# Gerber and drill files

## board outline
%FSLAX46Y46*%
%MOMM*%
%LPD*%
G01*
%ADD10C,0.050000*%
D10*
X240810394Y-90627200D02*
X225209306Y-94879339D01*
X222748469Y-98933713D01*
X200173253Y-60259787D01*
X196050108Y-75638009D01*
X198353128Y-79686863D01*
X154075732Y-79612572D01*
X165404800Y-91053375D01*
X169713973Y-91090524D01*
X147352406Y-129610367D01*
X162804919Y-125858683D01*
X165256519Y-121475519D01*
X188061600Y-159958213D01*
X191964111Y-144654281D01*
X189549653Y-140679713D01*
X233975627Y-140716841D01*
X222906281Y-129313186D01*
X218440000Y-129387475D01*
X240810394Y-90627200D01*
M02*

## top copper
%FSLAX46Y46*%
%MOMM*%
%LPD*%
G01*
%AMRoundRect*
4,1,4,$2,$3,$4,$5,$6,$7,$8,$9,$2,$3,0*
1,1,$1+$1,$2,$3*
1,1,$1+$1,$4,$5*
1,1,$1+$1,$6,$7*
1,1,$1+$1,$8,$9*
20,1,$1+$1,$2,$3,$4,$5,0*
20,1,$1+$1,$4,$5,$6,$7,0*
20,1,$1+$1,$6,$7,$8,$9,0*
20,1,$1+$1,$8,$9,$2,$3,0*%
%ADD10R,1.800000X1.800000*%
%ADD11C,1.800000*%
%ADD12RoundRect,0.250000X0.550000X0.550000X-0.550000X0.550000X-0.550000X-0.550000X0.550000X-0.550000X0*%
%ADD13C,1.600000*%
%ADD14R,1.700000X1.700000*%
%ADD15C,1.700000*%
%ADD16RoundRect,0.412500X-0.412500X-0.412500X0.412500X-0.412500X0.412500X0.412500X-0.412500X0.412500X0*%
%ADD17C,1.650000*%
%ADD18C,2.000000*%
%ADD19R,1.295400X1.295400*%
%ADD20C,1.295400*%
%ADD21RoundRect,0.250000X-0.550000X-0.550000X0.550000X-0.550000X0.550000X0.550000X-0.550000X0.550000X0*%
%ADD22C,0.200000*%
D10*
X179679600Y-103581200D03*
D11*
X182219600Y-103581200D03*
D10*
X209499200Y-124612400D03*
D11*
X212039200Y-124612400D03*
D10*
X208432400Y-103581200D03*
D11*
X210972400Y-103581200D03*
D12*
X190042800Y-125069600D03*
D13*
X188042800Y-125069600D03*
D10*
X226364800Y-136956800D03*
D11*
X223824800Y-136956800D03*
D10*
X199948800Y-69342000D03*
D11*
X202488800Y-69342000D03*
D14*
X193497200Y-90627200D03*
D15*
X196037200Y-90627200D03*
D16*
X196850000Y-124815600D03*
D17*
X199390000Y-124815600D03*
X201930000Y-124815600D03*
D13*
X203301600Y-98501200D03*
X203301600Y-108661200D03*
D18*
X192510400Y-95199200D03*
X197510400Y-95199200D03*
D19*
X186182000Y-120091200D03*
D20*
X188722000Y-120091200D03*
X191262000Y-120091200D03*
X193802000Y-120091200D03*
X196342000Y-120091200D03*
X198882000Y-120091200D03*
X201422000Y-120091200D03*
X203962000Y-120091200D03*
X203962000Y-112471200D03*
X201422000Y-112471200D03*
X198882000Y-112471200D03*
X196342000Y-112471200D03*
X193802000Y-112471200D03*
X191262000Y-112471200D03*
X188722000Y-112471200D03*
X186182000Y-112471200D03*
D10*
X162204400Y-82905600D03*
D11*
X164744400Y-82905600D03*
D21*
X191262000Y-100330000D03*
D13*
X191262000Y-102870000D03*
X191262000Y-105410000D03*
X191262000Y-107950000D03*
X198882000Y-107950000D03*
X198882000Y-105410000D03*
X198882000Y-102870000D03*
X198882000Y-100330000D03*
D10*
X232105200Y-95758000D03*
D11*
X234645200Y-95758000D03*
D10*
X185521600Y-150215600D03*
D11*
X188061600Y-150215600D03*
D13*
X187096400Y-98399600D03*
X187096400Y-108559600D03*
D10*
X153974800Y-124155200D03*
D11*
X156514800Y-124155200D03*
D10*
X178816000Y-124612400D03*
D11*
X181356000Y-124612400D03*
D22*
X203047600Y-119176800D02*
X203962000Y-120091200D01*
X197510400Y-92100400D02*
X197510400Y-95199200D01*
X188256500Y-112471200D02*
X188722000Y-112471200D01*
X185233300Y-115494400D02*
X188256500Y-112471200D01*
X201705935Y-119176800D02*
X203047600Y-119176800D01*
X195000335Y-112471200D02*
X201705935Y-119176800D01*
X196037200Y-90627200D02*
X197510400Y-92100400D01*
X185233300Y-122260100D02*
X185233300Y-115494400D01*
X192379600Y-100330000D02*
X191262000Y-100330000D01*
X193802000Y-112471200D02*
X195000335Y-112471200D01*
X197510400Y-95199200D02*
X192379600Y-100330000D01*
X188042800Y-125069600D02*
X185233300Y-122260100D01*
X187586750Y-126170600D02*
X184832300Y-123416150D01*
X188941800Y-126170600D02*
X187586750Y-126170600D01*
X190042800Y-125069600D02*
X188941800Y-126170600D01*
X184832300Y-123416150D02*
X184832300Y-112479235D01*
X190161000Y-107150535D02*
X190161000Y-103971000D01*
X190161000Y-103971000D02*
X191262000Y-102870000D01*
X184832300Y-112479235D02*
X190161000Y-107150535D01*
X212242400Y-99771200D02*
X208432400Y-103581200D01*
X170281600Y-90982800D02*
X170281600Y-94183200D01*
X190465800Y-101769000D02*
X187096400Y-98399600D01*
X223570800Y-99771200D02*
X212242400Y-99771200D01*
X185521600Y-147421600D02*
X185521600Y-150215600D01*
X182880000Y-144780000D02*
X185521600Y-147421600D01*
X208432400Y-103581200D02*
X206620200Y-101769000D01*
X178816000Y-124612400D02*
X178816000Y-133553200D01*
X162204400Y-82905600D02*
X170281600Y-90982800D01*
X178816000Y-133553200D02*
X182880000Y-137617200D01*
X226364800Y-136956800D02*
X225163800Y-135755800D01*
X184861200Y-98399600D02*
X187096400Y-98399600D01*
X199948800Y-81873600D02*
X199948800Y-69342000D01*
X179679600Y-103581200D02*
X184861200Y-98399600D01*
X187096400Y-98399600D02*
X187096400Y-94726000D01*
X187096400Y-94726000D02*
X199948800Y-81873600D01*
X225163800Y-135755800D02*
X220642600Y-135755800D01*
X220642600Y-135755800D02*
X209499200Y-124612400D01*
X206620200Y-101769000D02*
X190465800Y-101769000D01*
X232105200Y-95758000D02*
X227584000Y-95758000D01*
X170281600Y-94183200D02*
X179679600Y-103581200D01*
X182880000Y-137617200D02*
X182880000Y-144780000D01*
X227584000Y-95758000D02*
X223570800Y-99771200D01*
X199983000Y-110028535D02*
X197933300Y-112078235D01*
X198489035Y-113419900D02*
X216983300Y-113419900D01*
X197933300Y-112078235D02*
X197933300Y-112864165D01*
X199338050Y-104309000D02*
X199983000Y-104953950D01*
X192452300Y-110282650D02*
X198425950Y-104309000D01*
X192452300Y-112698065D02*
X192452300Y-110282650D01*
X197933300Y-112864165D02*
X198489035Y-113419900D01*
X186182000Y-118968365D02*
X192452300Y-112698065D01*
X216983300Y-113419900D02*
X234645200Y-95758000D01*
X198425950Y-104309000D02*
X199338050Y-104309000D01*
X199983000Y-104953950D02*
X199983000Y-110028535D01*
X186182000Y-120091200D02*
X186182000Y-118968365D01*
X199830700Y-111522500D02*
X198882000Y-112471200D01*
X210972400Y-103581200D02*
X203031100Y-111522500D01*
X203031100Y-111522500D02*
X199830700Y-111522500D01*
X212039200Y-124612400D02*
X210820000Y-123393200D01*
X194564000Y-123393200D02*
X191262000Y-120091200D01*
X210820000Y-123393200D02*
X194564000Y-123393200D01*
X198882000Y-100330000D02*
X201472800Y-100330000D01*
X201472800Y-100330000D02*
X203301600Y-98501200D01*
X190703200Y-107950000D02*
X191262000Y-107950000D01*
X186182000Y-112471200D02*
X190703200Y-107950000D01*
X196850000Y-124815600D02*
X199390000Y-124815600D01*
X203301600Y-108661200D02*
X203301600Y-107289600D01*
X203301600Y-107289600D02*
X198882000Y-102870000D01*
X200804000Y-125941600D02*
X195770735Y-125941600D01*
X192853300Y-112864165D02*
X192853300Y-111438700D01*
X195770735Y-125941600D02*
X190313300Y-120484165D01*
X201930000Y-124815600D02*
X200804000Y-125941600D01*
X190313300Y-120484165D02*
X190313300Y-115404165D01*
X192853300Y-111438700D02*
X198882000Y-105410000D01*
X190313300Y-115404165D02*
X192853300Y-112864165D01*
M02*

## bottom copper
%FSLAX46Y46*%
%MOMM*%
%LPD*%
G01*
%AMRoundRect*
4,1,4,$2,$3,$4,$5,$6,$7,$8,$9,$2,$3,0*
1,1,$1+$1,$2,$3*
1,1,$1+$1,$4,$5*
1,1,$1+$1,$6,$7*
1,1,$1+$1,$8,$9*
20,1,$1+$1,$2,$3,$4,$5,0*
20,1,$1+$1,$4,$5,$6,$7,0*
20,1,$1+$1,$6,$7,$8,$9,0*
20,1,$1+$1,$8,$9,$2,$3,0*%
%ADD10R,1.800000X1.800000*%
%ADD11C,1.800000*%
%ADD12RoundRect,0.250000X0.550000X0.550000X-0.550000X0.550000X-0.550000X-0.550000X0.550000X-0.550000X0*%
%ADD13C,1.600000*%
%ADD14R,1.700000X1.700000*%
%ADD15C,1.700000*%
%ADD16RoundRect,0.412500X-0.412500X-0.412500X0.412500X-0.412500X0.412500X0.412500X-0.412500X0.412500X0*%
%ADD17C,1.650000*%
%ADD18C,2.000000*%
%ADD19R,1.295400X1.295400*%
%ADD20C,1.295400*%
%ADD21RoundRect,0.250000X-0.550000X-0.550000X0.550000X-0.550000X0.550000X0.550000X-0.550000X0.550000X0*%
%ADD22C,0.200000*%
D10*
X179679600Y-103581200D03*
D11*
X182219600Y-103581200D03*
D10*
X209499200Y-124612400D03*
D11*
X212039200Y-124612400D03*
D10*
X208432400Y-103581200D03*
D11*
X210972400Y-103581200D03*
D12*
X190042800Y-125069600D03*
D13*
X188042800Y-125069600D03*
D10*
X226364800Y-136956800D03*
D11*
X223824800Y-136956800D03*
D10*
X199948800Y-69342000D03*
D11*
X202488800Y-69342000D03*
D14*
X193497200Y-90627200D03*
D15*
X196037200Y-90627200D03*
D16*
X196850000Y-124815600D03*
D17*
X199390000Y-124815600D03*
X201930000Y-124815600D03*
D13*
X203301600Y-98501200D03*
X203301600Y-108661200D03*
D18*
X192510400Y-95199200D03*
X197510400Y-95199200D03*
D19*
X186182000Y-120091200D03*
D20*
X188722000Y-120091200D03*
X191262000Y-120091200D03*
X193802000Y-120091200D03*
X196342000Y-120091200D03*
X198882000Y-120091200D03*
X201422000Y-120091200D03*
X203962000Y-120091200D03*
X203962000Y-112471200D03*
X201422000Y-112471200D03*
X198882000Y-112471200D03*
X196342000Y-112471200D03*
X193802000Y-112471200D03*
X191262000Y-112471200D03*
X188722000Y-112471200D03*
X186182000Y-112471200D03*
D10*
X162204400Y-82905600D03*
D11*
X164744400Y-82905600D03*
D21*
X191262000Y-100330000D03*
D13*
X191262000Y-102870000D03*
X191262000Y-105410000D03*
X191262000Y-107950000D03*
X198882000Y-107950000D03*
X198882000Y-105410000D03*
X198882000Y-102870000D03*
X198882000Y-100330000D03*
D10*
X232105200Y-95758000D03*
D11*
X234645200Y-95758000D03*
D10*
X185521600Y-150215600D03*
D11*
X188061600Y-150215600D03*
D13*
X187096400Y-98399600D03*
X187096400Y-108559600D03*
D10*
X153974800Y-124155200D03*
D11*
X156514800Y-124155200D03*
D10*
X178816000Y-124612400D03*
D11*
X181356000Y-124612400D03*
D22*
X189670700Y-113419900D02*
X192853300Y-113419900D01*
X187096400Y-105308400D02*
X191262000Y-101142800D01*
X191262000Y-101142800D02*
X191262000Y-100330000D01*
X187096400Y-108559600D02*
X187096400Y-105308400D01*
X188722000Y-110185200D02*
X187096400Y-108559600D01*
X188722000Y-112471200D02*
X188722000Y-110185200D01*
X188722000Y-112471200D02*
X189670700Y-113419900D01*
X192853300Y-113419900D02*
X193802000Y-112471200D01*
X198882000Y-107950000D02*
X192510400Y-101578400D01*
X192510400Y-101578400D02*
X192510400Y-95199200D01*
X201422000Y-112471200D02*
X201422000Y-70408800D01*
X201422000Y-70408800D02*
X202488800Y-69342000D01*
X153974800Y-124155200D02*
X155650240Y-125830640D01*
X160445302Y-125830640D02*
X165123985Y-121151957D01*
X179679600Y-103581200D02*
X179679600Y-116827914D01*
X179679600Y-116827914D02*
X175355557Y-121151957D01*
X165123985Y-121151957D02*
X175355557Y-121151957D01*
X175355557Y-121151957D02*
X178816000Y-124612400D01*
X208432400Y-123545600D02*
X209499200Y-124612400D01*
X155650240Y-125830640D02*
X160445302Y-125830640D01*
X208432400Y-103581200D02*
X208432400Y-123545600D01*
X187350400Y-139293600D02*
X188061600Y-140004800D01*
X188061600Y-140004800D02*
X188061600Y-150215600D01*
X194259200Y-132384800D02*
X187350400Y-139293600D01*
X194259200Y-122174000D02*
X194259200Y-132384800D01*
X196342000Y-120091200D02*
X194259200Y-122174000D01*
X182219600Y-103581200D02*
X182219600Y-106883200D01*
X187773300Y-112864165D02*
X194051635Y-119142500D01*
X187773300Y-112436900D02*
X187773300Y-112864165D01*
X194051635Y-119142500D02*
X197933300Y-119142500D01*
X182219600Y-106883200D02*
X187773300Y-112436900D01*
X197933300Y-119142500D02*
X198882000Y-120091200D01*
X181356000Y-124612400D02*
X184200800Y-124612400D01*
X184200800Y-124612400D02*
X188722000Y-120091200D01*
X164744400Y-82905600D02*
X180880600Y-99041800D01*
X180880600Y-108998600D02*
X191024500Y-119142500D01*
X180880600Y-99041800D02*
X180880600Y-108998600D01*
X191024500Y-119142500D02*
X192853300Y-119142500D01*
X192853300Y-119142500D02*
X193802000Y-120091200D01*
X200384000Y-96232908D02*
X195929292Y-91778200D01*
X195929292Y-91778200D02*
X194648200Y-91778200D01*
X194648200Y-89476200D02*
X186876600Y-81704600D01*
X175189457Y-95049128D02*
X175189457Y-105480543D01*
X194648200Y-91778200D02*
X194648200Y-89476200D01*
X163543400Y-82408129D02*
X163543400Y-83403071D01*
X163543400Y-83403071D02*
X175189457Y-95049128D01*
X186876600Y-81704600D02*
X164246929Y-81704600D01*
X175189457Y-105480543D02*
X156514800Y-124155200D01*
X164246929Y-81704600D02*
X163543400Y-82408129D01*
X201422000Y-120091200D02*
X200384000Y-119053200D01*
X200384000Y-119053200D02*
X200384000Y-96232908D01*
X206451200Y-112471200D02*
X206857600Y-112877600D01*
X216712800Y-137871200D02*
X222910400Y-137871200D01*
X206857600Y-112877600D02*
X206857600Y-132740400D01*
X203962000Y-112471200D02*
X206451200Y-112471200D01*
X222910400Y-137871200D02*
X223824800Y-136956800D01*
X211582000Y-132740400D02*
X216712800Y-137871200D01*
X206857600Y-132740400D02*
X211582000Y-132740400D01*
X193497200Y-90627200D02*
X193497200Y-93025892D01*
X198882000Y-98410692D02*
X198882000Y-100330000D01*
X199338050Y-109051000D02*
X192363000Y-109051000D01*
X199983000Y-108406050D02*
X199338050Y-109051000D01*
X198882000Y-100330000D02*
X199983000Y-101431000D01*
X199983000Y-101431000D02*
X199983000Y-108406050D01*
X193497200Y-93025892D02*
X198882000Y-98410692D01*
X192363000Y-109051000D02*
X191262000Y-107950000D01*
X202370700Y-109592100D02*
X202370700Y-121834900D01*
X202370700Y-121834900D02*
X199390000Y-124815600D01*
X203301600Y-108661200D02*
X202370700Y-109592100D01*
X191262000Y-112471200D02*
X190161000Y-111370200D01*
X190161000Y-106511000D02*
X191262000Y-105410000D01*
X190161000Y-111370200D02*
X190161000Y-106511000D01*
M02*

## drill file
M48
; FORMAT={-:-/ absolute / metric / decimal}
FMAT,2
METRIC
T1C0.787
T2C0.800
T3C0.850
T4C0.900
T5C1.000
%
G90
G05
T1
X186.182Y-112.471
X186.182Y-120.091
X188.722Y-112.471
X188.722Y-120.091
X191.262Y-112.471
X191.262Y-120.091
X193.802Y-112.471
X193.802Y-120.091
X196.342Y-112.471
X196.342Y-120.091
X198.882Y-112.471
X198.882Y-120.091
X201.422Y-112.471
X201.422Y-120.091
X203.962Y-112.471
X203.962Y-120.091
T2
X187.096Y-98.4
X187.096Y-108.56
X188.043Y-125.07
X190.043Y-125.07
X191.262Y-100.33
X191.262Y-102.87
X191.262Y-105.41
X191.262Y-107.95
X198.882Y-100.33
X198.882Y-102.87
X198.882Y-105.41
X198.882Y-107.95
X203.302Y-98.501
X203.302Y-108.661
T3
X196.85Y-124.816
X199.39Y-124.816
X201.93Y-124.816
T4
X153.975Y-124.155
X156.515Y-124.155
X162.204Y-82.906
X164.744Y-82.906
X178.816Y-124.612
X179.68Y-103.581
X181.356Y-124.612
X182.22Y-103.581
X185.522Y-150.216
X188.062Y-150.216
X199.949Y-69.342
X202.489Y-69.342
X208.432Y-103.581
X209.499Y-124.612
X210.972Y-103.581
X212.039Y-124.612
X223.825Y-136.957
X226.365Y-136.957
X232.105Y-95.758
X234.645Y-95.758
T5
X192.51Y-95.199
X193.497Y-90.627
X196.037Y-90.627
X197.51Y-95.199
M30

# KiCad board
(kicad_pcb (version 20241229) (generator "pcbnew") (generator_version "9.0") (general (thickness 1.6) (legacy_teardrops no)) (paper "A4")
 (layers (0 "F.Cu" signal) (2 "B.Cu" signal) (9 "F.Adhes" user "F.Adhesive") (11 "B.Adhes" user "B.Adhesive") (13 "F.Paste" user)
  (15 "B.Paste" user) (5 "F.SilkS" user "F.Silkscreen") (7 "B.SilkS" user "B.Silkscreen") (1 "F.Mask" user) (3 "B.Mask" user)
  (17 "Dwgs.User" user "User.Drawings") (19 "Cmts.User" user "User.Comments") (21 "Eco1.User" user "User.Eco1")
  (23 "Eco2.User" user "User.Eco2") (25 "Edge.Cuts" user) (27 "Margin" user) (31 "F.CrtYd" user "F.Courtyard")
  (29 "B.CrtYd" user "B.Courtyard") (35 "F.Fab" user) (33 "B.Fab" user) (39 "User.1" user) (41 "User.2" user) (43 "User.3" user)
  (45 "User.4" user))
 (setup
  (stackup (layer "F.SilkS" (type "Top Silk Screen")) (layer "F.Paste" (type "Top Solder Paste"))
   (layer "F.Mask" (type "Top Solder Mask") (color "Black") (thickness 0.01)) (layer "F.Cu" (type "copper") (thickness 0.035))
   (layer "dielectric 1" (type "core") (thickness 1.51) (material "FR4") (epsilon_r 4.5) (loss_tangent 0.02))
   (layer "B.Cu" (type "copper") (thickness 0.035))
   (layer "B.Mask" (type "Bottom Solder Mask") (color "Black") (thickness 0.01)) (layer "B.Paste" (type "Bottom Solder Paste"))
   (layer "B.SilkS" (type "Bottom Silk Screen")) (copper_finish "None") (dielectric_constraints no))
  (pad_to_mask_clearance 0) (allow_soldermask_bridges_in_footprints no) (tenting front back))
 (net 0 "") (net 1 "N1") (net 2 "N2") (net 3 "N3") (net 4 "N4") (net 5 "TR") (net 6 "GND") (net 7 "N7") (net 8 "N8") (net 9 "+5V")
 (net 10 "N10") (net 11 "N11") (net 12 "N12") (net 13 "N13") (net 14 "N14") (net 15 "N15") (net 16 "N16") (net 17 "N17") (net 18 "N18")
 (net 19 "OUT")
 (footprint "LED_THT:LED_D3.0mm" (layer "F.Cu") (at 179.6796 103.5812)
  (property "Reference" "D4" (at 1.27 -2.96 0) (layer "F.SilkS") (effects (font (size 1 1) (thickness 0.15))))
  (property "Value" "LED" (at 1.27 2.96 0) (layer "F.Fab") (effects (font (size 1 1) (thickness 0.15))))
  (pad "1" thru_hole rect (at 0 0) (size 1.8 1.8) (drill 0.9) (layers "*.Cu" "*.Mask") (remove_unused_layers no) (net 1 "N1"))
  (pad "2" thru_hole circle (at 2.54 0) (size 1.8 1.8) (drill 0.9) (layers "*.Cu" "*.Mask") (remove_unused_layers no) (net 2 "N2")))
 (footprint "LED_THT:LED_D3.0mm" (layer "F.Cu") (at 209.4992 124.6124)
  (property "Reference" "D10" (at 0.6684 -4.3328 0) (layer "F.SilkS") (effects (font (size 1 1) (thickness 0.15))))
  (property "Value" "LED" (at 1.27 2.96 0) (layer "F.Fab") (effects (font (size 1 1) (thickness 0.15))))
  (pad "1" thru_hole rect (at 0 0) (size 1.8 1.8) (drill 0.9) (layers "*.Cu" "*.Mask") (remove_unused_layers no) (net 1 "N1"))
  (pad "2" thru_hole circle (at 2.54 0) (size 1.8 1.8) (drill 0.9) (layers "*.Cu" "*.Mask") (remove_unused_layers no) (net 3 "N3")))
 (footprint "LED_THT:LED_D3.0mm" (layer "F.Cu") (at 208.4324 103.5812)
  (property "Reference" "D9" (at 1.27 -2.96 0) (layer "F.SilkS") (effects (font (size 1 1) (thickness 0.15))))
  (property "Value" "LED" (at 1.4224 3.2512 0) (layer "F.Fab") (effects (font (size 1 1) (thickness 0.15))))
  (pad "1" thru_hole rect (at 0 0) (size 1.8 1.8) (drill 0.9) (layers "*.Cu" "*.Mask") (remove_unused_layers no) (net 1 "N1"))
  (pad "2" thru_hole circle (at 2.54 0) (size 1.8 1.8) (drill 0.9) (layers "*.Cu" "*.Mask") (remove_unused_layers no) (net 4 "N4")))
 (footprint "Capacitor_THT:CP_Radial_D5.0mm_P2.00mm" (layer "F.Cu") (at 190.0428 125.0696 180)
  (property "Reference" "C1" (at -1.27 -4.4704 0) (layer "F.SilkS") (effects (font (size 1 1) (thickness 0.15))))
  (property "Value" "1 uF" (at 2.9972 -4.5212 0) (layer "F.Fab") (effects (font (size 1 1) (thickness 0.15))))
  (pad "1" thru_hole roundrect (at 0 0 180) (size 1.6 1.6) (drill 0.8) (layers "*.Cu" "*.Mask") (remove_unused_layers no)
   (roundrect_rratio 0.15625) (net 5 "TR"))
  (pad "2" thru_hole circle (at 2 0 180) (size 1.6 1.6) (drill 0.8) (layers "*.Cu" "*.Mask") (remove_unused_layers no) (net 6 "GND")))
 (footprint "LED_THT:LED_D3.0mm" (layer "F.Cu") (at 226.3648 136.9568 180)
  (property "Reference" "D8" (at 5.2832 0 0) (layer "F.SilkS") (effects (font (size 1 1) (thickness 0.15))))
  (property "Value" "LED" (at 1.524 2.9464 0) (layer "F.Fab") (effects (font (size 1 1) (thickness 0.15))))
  (pad "1" thru_hole rect (at 0 0 180) (size 1.8 1.8) (drill 0.9) (layers "*.Cu" "*.Mask") (remove_unused_layers no) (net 1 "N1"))
  (pad "2" thru_hole circle (at 2.54 0 180) (size 1.8 1.8) (drill 0.9) (layers "*.Cu" "*.Mask") (remove_unused_layers no) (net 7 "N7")))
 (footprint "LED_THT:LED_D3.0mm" (layer "F.Cu") (at 199.9488 69.342)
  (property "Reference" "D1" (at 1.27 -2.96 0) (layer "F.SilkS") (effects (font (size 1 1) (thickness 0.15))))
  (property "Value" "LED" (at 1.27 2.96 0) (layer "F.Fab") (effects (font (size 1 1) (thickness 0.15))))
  (pad "1" thru_hole rect (at 0 0) (size 1.8 1.8) (drill 0.9) (layers "*.Cu" "*.Mask") (remove_unused_layers no) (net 1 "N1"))
  (pad "2" thru_hole circle (at 2.54 0) (size 1.8 1.8) (drill 0.9) (layers "*.Cu" "*.Mask") (remove_unused_layers no) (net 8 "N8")))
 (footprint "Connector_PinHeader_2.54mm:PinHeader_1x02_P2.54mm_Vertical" (layer "F.Cu") (at 193.4972 90.6272 90)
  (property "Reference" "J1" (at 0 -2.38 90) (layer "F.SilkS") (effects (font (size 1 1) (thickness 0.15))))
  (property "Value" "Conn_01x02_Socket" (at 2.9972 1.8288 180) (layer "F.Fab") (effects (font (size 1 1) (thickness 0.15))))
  (pad "1" thru_hole rect (at 0 0 90) (size 1.7 1.7) (drill 1) (layers "*.Cu" "*.Mask") (remove_unused_layers no) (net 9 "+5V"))
  (pad "2" thru_hole circle (at 0 2.54 90) (size 1.7 1.7) (drill 1) (layers "*.Cu" "*.Mask") (remove_unused_layers no) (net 6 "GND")))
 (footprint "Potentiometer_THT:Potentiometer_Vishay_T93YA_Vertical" (layer "F.Cu") (at 196.85 124.8156)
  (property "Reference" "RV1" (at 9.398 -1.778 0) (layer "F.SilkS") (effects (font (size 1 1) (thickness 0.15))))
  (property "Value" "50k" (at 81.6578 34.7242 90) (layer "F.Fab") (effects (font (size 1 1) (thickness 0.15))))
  (pad "1" thru_hole roundrect (at 0 0) (size 1.65 1.65) (drill 0.85) (layers "*.Cu" "*.Mask") (remove_unused_layers no)
   (roundrect_rratio 0.25) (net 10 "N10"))
  (pad "2" thru_hole circle (at 2.54 0) (size 1.65 1.65) (drill 0.85) (layers "*.Cu" "*.Mask") (remove_unused_layers no) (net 10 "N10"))
  (pad "3" thru_hole circle (at 5.08 0) (size 1.65 1.65) (drill 0.85) (layers "*.Cu" "*.Mask") (remove_unused_layers no) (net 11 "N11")))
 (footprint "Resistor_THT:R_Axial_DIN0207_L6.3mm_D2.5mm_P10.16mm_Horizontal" (layer "F.Cu") (at 203.3016 98.5012 -90)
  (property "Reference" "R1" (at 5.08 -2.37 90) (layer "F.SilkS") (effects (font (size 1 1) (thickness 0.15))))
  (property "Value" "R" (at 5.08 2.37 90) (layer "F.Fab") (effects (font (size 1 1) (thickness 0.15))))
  (pad "1" thru_hole circle (at 0 0 270) (size 1.6 1.6) (drill 0.8) (layers "*.Cu" "*.Mask") (remove_unused_layers no) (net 9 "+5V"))
  (pad "2" thru_hole circle (at 10.16 0 270) (size 1.6 1.6) (drill 0.8) (layers "*.Cu" "*.Mask") (remove_unused_layers no) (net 10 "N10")))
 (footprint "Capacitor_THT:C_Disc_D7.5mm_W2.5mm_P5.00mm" (layer "F.Cu") (at 192.5104 95.1992)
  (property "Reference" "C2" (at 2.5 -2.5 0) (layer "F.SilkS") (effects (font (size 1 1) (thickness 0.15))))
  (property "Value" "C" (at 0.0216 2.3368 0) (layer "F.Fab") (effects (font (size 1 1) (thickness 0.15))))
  (pad "1" thru_hole circle (at 0 0) (size 2 2) (drill 1) (layers "*.Cu" "*.Mask") (remove_unused_layers no) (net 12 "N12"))
  (pad "2" thru_hole circle (at 5 0) (size 2 2) (drill 1) (layers "*.Cu" "*.Mask") (remove_unused_layers no) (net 6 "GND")))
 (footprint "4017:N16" (layer "F.Cu") (at 203.962 112.4712 90)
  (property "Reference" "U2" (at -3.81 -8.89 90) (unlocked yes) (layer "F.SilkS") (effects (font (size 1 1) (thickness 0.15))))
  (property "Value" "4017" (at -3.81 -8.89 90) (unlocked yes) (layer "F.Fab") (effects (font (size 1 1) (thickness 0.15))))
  (pad "1" thru_hole rect (at -7.62 -17.78 90) (size 1.2954 1.2954) (drill 0.7874) (layers "*.Cu" "*.Mask") (remove_unused_layers no)
   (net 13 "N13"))
  (pad "2" thru_hole circle (at -7.62 -15.24 90) (size 1.2954 1.2954) (drill 0.7874) (layers "*.Cu" "*.Mask") (remove_unused_layers no)
   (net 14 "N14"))
  (pad "3" thru_hole circle (at -7.62 -12.7 90) (size 1.2954 1.2954) (drill 0.7874) (layers "*.Cu" "*.Mask") (remove_unused_layers no)
   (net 3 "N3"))
  (pad "4" thru_hole circle (at -7.62 -10.16 90) (size 1.2954 1.2954) (drill 0.7874) (layers "*.Cu" "*.Mask") (remove_unused_layers no)
   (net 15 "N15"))
  (pad "5" thru_hole circle (at -7.62 -7.62 90) (size 1.2954 1.2954) (drill 0.7874) (layers "*.Cu" "*.Mask") (remove_unused_layers no)
   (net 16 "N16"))
  (pad "6" thru_hole circle (at -7.62 -5.08 90) (size 1.2954 1.2954) (drill 0.7874) (layers "*.Cu" "*.Mask") (remove_unused_layers no)
   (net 2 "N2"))
  (pad "7" thru_hole circle (at -7.62 -2.54 90) (size 1.2954 1.2954) (drill 0.7874) (layers "*.Cu" "*.Mask") (remove_unused_layers no)
   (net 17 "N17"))
  (pad "8" thru_hole circle (at -7.62 0 90) (size 1.2954 1.2954) (drill 0.7874) (layers "*.Cu" "*.Mask") (remove_unused_layers no)
   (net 6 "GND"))
  (pad "9" thru_hole circle (at 0 0 90) (size 1.2954 1.2954) (drill 0.7874) (layers "*.Cu" "*.Mask") (remove_unused_layers no) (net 7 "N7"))
  (pad "10" thru_hole circle (at 0 -2.54 90) (size 1.2954 1.2954) (drill 0.7874) (layers "*.Cu" "*.Mask") (remove_unused_layers no)
   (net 8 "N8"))
  (pad "11" thru_hole circle (at 0 -5.08 90) (size 1.2954 1.2954) (drill 0.7874) (layers "*.Cu" "*.Mask") (remove_unused_layers no)
   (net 4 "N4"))
  (pad "12" thru_hole circle (at 0 -7.62 90) (size 1.2954 1.2954) (drill 0.7874) (layers "*.Cu" "*.Mask") (remove_unused_layers no)
   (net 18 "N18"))
  (pad "13" thru_hole circle (at 0 -10.16 90) (size 1.2954 1.2954) (drill 0.7874) (layers "*.Cu" "*.Mask") (remove_unused_layers no)
   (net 6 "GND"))
  (pad "14" thru_hole circle (at 0 -12.7 90) (size 1.2954 1.2954) (drill 0.7874) (layers "*.Cu" "*.Mask") (remove_unused_layers no)
   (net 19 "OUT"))
  (pad "15" thru_hole circle (at 0 -15.24 90) (size 1.2954 1.2954) (drill 0.7874) (layers "*.Cu" "*.Mask") (remove_unused_layers no)
   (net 6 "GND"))
  (pad "16" thru_hole circle (at 0 -17.78 90) (size 1.2954 1.2954) (drill 0.7874) (layers "*.Cu" "*.Mask") (remove_unused_layers no)
   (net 9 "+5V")))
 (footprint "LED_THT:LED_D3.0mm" (layer "F.Cu") (at 162.2044 82.9056)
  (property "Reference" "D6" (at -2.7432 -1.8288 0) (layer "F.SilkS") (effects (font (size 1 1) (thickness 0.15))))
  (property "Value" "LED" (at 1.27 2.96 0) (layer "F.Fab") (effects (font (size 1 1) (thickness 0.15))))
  (pad "1" thru_hole rect (at 0 0) (size 1.8 1.8) (drill 0.9) (layers "*.Cu" "*.Mask") (remove_unused_layers no) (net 1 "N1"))
  (pad "2" thru_hole circle (at 2.54 0) (size 1.8 1.8) (drill 0.9) (layers "*.Cu" "*.Mask") (remove_unused_layers no) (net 15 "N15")))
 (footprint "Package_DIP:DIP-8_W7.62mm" (layer "F.Cu") (at 191.262 100.33)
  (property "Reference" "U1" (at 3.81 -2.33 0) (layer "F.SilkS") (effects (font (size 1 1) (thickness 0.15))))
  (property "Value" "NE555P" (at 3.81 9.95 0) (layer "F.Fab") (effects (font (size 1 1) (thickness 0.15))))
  (pad "1" thru_hole roundrect (at 0 0) (size 1.6 1.6) (drill 0.8) (layers "*.Cu" "*.Mask") (remove_unused_layers no)
   (roundrect_rratio 0.15625) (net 6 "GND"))
  (pad "2" thru_hole circle (at 0 2.54) (size 1.6 1.6) (drill 0.8) (layers "*.Cu" "*.Mask") (remove_unused_layers no) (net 5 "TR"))
  (pad "3" thru_hole circle (at 0 5.08) (size 1.6 1.6) (drill 0.8) (layers "*.Cu" "*.Mask") (remove_unused_layers no) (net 19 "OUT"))
  (pad "4" thru_hole circle (at 0 7.62) (size 1.6 1.6) (drill 0.8) (layers "*.Cu" "*.Mask") (remove_unused_layers no) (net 9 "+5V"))
  (pad "5" thru_hole circle (at 7.62 7.62) (size 1.6 1.6) (drill 0.8) (layers "*.Cu" "*.Mask") (remove_unused_layers no) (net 12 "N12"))
  (pad "6" thru_hole circle (at 7.62 5.08) (size 1.6 1.6) (drill 0.8) (layers "*.Cu" "*.Mask") (remove_unused_layers no) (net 11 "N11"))
  (pad "7" thru_hole circle (at 7.62 2.54) (size 1.6 1.6) (drill 0.8) (layers "*.Cu" "*.Mask") (remove_unused_layers no) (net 10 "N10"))
  (pad "8" thru_hole circle (at 7.62 0) (size 1.6 1.6) (drill 0.8) (layers "*.Cu" "*.Mask") (remove_unused_layers no) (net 9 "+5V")))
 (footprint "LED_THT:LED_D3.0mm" (layer "F.Cu") (at 232.1052 95.758)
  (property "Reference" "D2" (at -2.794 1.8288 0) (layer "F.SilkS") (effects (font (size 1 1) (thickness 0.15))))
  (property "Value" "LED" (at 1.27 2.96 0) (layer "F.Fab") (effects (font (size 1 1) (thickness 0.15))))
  (pad "1" thru_hole rect (at 0 0) (size 1.8 1.8) (drill 0.9) (layers "*.Cu" "*.Mask") (remove_unused_layers no) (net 1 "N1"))
  (pad "2" thru_hole circle (at 2.54 0) (size 1.8 1.8) (drill 0.9) (layers "*.Cu" "*.Mask") (remove_unused_layers no) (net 13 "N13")))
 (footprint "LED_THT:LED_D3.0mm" (layer "F.Cu") (at 185.5216 150.2156)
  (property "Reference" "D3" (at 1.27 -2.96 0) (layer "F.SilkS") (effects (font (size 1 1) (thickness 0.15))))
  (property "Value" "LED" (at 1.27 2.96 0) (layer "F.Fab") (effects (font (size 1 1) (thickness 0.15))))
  (pad "1" thru_hole rect (at 0 0) (size 1.8 1.8) (drill 0.9) (layers "*.Cu" "*.Mask") (remove_unused_layers no) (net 1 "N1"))
  (pad "2" thru_hole circle (at 2.54 0) (size 1.8 1.8) (drill 0.9) (layers "*.Cu" "*.Mask") (remove_unused_layers no) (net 16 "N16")))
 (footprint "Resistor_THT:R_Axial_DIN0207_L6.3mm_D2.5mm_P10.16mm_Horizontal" (layer "F.Cu") (at 187.0964 98.3996 -90)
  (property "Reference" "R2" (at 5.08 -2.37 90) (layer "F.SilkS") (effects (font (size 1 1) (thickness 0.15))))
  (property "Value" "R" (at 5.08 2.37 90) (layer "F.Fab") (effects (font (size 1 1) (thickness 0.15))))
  (pad "1" thru_hole circle (at 0 0 270) (size 1.6 1.6) (drill 0.8) (layers "*.Cu" "*.Mask") (remove_unused_layers no) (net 1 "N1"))
  (pad "2" thru_hole circle (at 10.16 0 270) (size 1.6 1.6) (drill 0.8) (layers "*.Cu" "*.Mask") (remove_unused_layers no) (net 6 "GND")))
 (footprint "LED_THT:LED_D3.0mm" (layer "F.Cu") (at 153.9748 124.1552)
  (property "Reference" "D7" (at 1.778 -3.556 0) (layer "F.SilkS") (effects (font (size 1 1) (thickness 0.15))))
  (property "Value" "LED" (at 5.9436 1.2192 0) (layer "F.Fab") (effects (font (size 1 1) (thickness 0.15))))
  (pad "1" thru_hole rect (at 0 0) (size 1.8 1.8) (drill 0.9) (layers "*.Cu" "*.Mask") (remove_unused_layers no) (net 1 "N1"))
  (pad "2" thru_hole circle (at 2.54 0) (size 1.8 1.8) (drill 0.9) (layers "*.Cu" "*.Mask") (remove_unused_layers no) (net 17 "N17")))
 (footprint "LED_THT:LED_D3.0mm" (layer "F.Cu") (at 178.816 124.6124)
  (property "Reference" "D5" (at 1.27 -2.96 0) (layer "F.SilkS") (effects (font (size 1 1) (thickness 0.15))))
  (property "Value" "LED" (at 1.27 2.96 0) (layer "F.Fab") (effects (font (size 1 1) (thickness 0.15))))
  (pad "1" thru_hole rect (at 0 0) (size 1.8 1.8) (drill 0.9) (layers "*.Cu" "*.Mask") (remove_unused_layers no) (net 1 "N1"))
  (pad "2" thru_hole circle (at 2.54 0) (size 1.8 1.8) (drill 0.9) (layers "*.Cu" "*.Mask") (remove_unused_layers no) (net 14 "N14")))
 (gr_poly
  (pts (xy 240.810394 90.6272) (xy 225.209306 94.879339) (xy 222.748469 98.933713) (xy 200.173253 60.259787) (xy 196.050108 75.638009)
   (xy 198.353128 79.686863) (xy 154.075732 79.612572) (xy 165.4048 91.053375) (xy 169.713973 91.090524) (xy 147.352406 129.610367)
   (xy 162.804919 125.858683) (xy 165.256519 121.475519) (xy 188.0616 159.958213) (xy 191.964111 144.654281) (xy 189.549653 140.679713)
   (xy 233.975627 140.716841) (xy 222.906281 129.313186) (xy 218.44 129.387475))
  (stroke (width 0.05) (type solid)) (fill no) (layer "Edge.Cuts"))
 (segment (start 203.0476 119.1768) (end 203.962 120.0912) (width 0.2) (layer "F.Cu") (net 6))
 (segment (start 197.5104 92.1004) (end 197.5104 95.1992) (width 0.2) (layer "F.Cu") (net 6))
 (segment (start 188.2565 112.4712) (end 188.722 112.4712) (width 0.2) (layer "F.Cu") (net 6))
 (segment (start 185.2333 115.4944) (end 188.2565 112.4712) (width 0.2) (layer "F.Cu") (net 6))
 (segment (start 201.705935 119.1768) (end 203.0476 119.1768) (width 0.2) (layer "F.Cu") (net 6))
 (segment (start 195.000335 112.4712) (end 201.705935 119.1768) (width 0.2) (layer "F.Cu") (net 6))
 (segment (start 196.0372 90.6272) (end 197.5104 92.1004) (width 0.2) (layer "F.Cu") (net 6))
 (segment (start 185.2333 122.2601) (end 185.2333 115.4944) (width 0.2) (layer "F.Cu") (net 6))
 (segment (start 192.3796 100.33) (end 191.262 100.33) (width 0.2) (layer "F.Cu") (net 6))
 (segment (start 193.802 112.4712) (end 195.000335 112.4712) (width 0.2) (layer "F.Cu") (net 6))
 (segment (start 197.5104 95.1992) (end 192.3796 100.33) (width 0.2) (layer "F.Cu") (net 6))
 (segment (start 188.0428 125.0696) (end 185.2333 122.2601) (width 0.2) (layer "F.Cu") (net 6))
 (segment (start 189.6707 113.4199) (end 192.8533 113.4199) (width 0.2) (layer "B.Cu") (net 6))
 (segment (start 187.0964 105.3084) (end 191.262 101.1428) (width 0.2) (layer "B.Cu") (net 6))
 (segment (start 191.262 101.1428) (end 191.262 100.33) (width 0.2) (layer "B.Cu") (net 6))
 (segment (start 187.0964 108.5596) (end 187.0964 105.3084) (width 0.2) (layer "B.Cu") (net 6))
 (segment (start 188.722 110.1852) (end 187.0964 108.5596) (width 0.2) (layer "B.Cu") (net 6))
 (segment (start 188.722 112.4712) (end 188.722 110.1852) (width 0.2) (layer "B.Cu") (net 6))
 (segment (start 188.722 112.4712) (end 189.6707 113.4199) (width 0.2) (layer "B.Cu") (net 6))
 (segment (start 192.8533 113.4199) (end 193.802 112.4712) (width 0.2) (layer "B.Cu") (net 6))
 (segment (start 187.58675 126.1706) (end 184.8323 123.41615) (width 0.2) (layer "F.Cu") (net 5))
 (segment (start 188.9418 126.1706) (end 187.58675 126.1706) (width 0.2) (layer "F.Cu") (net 5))
 (segment (start 190.0428 125.0696) (end 188.9418 126.1706) (width 0.2) (layer "F.Cu") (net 5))
 (segment (start 184.8323 123.41615) (end 184.8323 112.479235) (width 0.2) (layer "F.Cu") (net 5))
 (segment (start 190.161 107.150535) (end 190.161 103.971) (width 0.2) (layer "F.Cu") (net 5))
 (segment (start 190.161 103.971) (end 191.262 102.87) (width 0.2) (layer "F.Cu") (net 5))
 (segment (start 184.8323 112.479235) (end 190.161 107.150535) (width 0.2) (layer "F.Cu") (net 5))
 (segment (start 198.882 107.95) (end 192.5104 101.5784) (width 0.2) (layer "B.Cu") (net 12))
 (segment (start 192.5104 101.5784) (end 192.5104 95.1992) (width 0.2) (layer "B.Cu") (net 12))
 (segment (start 201.422 112.4712) (end 201.422 70.4088) (width 0.2) (layer "B.Cu") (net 8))
 (segment (start 201.422 70.4088) (end 202.4888 69.342) (width 0.2) (layer "B.Cu") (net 8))
 (segment (start 212.2424 99.7712) (end 208.4324 103.5812) (width 0.2) (layer "F.Cu") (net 1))
 (segment (start 170.2816 90.9828) (end 170.2816 94.1832) (width 0.2) (layer "F.Cu") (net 1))
 (segment (start 190.4658 101.769) (end 187.0964 98.3996) (width 0.2) (layer "F.Cu") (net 1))
 (segment (start 223.5708 99.7712) (end 212.2424 99.7712) (width 0.2) (layer "F.Cu") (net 1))
 (segment (start 185.5216 147.4216) (end 185.5216 150.2156) (width 0.2) (layer "F.Cu") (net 1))
 (segment (start 182.88 144.78) (end 185.5216 147.4216) (width 0.2) (layer "F.Cu") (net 1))
 (segment (start 208.4324 103.5812) (end 206.6202 101.769) (width 0.2) (layer "F.Cu") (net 1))
 (segment (start 178.816 124.6124) (end 178.816 133.5532) (width 0.2) (layer "F.Cu") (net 1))
 (segment (start 162.2044 82.9056) (end 170.2816 90.9828) (width 0.2) (layer "F.Cu") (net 1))
 (segment (start 178.816 133.5532) (end 182.88 137.6172) (width 0.2) (layer "F.Cu") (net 1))
 (segment (start 226.3648 136.9568) (end 225.1638 135.7558) (width 0.2) (layer "F.Cu") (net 1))
 (segment (start 184.8612 98.3996) (end 187.0964 98.3996) (width 0.2) (layer "F.Cu") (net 1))
 (segment (start 199.9488 81.8736) (end 199.9488 69.342) (width 0.2) (layer "F.Cu") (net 1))
 (segment (start 179.6796 103.5812) (end 184.8612 98.3996) (width 0.2) (layer "F.Cu") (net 1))
 (segment (start 187.0964 98.3996) (end 187.0964 94.726) (width 0.2) (layer "F.Cu") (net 1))
 (segment (start 187.0964 94.726) (end 199.9488 81.8736) (width 0.2) (layer "F.Cu") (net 1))
 (segment (start 225.1638 135.7558) (end 220.6426 135.7558) (width 0.2) (layer "F.Cu") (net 1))
 (segment (start 220.6426 135.7558) (end 209.4992 124.6124) (width 0.2) (layer "F.Cu") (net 1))
 (segment (start 206.6202 101.769) (end 190.4658 101.769) (width 0.2) (layer "F.Cu") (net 1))
 (segment (start 232.1052 95.758) (end 227.584 95.758) (width 0.2) (layer "F.Cu") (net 1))
 (segment (start 170.2816 94.1832) (end 179.6796 103.5812) (width 0.2) (layer "F.Cu") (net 1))
 (segment (start 182.88 137.6172) (end 182.88 144.78) (width 0.2) (layer "F.Cu") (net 1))
 (segment (start 227.584 95.758) (end 223.5708 99.7712) (width 0.2) (layer "F.Cu") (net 1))
 (segment (start 153.9748 124.1552) (end 155.65024 125.83064) (width 0.2) (layer "B.Cu") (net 1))
 (segment (start 160.445302 125.83064) (end 165.123985 121.151957) (width 0.2) (layer "B.Cu") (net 1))
 (segment (start 179.6796 103.5812) (end 179.6796 116.827914) (width 0.2) (layer "B.Cu") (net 1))
 (segment (start 179.6796 116.827914) (end 175.355557 121.151957) (width 0.2) (layer "B.Cu") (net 1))
 (segment (start 165.123985 121.151957) (end 175.355557 121.151957) (width 0.2) (layer "B.Cu") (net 1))
 (segment (start 175.355557 121.151957) (end 178.816 124.6124) (width 0.2) (layer "B.Cu") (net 1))
 (segment (start 208.4324 123.5456) (end 209.4992 124.6124) (width 0.2) (layer "B.Cu") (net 1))
 (segment (start 155.65024 125.83064) (end 160.445302 125.83064) (width 0.2) (layer "B.Cu") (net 1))
 (segment (start 208.4324 103.5812) (end 208.4324 123.5456) (width 0.2) (layer "B.Cu") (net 1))
 (segment (start 199.983 110.028535) (end 197.9333 112.078235) (width 0.2) (layer "F.Cu") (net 13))
 (segment (start 198.489035 113.4199) (end 216.9833 113.4199) (width 0.2) (layer "F.Cu") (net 13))
 (segment (start 197.9333 112.078235) (end 197.9333 112.864165) (width 0.2) (layer "F.Cu") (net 13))
 (segment (start 199.33805 104.309) (end 199.983 104.95395) (width 0.2) (layer "F.Cu") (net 13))
 (segment (start 192.4523 110.28265) (end 198.42595 104.309) (width 0.2) (layer "F.Cu") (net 13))
 (segment (start 192.4523 112.698065) (end 192.4523 110.28265) (width 0.2) (layer "F.Cu") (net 13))
 (segment (start 197.9333 112.864165) (end 198.489035 113.4199) (width 0.2) (layer "F.Cu") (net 13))
 (segment (start 186.182 118.968365) (end 192.4523 112.698065) (width 0.2) (layer "F.Cu") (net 13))
 (segment (start 216.9833 113.4199) (end 234.6452 95.758) (width 0.2) (layer "F.Cu") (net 13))
 (segment (start 198.42595 104.309) (end 199.33805 104.309) (width 0.2) (layer "F.Cu") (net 13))
 (segment (start 199.983 104.95395) (end 199.983 110.028535) (width 0.2) (layer "F.Cu") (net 13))
 (segment (start 186.182 120.0912) (end 186.182 118.968365) (width 0.2) (layer "F.Cu") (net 13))
 (segment (start 187.3504 139.2936) (end 188.0616 140.0048) (width 0.2) (layer "B.Cu") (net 16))
 (segment (start 188.0616 140.0048) (end 188.0616 150.2156) (width 0.2) (layer "B.Cu") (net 16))
 (segment (start 194.2592 132.3848) (end 187.3504 139.2936) (width 0.2) (layer "B.Cu") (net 16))
 (segment (start 194.2592 122.174) (end 194.2592 132.3848) (width 0.2) (layer "B.Cu") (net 16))
 (segment (start 196.342 120.0912) (end 194.2592 122.174) (width 0.2) (layer "B.Cu") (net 16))
 (segment (start 182.2196 103.5812) (end 182.2196 106.8832) (width 0.2) (layer "B.Cu") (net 2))
 (segment (start 187.7733 112.864165) (end 194.051635 119.1425) (width 0.2) (layer "B.Cu") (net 2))
 (segment (start 187.7733 112.4369) (end 187.7733 112.864165) (width 0.2) (layer "B.Cu") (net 2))
 (segment (start 194.051635 119.1425) (end 197.9333 119.1425) (width 0.2) (layer "B.Cu") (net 2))
 (segment (start 182.2196 106.8832) (end 187.7733 112.4369) (width 0.2) (layer "B.Cu") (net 2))
 (segment (start 197.9333 119.1425) (end 198.882 120.0912) (width 0.2) (layer "B.Cu") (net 2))
 (segment (start 181.356 124.6124) (end 184.2008 124.6124) (width 0.2) (layer "B.Cu") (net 14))
 (segment (start 184.2008 124.6124) (end 188.722 120.0912) (width 0.2) (layer "B.Cu") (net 14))
 (segment (start 164.7444 82.9056) (end 180.8806 99.0418) (width 0.2) (layer "B.Cu") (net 15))
 (segment (start 180.8806 108.9986) (end 191.0245 119.1425) (width 0.2) (layer "B.Cu") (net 15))
 (segment (start 180.8806 99.0418) (end 180.8806 108.9986) (width 0.2) (layer "B.Cu") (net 15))
 (segment (start 191.0245 119.1425) (end 192.8533 119.1425) (width 0.2) (layer "B.Cu") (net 15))
 (segment (start 192.8533 119.1425) (end 193.802 120.0912) (width 0.2) (layer "B.Cu") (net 15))
 (segment (start 200.384 96.232908) (end 195.929292 91.7782) (width 0.2) (layer "B.Cu") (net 17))
 (segment (start 195.929292 91.7782) (end 194.6482 91.7782) (width 0.2) (layer "B.Cu") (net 17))
 (segment (start 194.6482 89.4762) (end 186.8766 81.7046) (width 0.2) (layer "B.Cu") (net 17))
 (segment (start 175.189457 95.049128) (end 175.189457 105.480543) (width 0.2) (layer "B.Cu") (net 17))
 (segment (start 194.6482 91.7782) (end 194.6482 89.4762) (width 0.2) (layer "B.Cu") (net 17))
 (segment (start 163.5434 82.408129) (end 163.5434 83.403071) (width 0.2) (layer "B.Cu") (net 17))
 (segment (start 163.5434 83.403071) (end 175.189457 95.049128) (width 0.2) (layer "B.Cu") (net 17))
 (segment (start 186.8766 81.7046) (end 164.246929 81.7046) (width 0.2) (layer "B.Cu") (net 17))
 (segment (start 175.189457 105.480543) (end 156.5148 124.1552) (width 0.2) (layer "B.Cu") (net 17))
 (segment (start 164.246929 81.7046) (end 163.5434 82.408129) (width 0.2) (layer "B.Cu") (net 17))
 (segment (start 201.422 120.0912) (end 200.384 119.0532) (width 0.2) (layer "B.Cu") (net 17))
 (segment (start 200.384 119.0532) (end 200.384 96.232908) (width 0.2) (layer "B.Cu") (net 17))
 (segment (start 206.4512 112.4712) (end 206.8576 112.8776) (width 0.2) (layer "B.Cu") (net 7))
 (segment (start 216.7128 137.8712) (end 222.9104 137.8712) (width 0.2) (layer "B.Cu") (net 7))
 (segment (start 206.8576 112.8776) (end 206.8576 132.7404) (width 0.2) (layer "B.Cu") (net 7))
 (segment (start 203.962 112.4712) (end 206.4512 112.4712) (width 0.2) (layer "B.Cu") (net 7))
 (segment (start 222.9104 137.8712) (end 223.8248 136.9568) (width 0.2) (layer "B.Cu") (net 7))
 (segment (start 211.582 132.7404) (end 216.7128 137.8712) (width 0.2) (layer "B.Cu") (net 7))
 (segment (start 206.8576 132.7404) (end 211.582 132.7404) (width 0.2) (layer "B.Cu") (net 7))
 (segment (start 199.8307 111.5225) (end 198.882 112.4712) (width 0.2) (layer "F.Cu") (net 4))
 (segment (start 210.9724 103.5812) (end 203.0311 111.5225) (width 0.2) (layer "F.Cu") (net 4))
 (segment (start 203.0311 111.5225) (end 199.8307 111.5225) (width 0.2) (layer "F.Cu") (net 4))
 (segment (start 212.0392 124.6124) (end 210.82 123.3932) (width 0.2) (layer "F.Cu") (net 3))
 (segment (start 194.564 123.3932) (end 191.262 120.0912) (width 0.2) (layer "F.Cu") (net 3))
 (segment (start 210.82 123.3932) (end 194.564 123.3932) (width 0.2) (layer "F.Cu") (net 3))
 (segment (start 198.882 100.33) (end 201.4728 100.33) (width 0.2) (layer "F.Cu") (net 9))
 (segment (start 201.4728 100.33) (end 203.3016 98.5012) (width 0.2) (layer "F.Cu") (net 9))
 (segment (start 190.7032 107.95) (end 191.262 107.95) (width 0.2) (layer "F.Cu") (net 9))
 (segment (start 186.182 112.4712) (end 190.7032 107.95) (width 0.2) (layer "F.Cu") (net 9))
 (segment (start 193.4972 90.6272) (end 193.4972 93.025892) (width 0.2) (layer "B.Cu") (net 9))
 (segment (start 198.882 98.410692) (end 198.882 100.33) (width 0.2) (layer "B.Cu") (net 9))
 (segment (start 199.33805 109.051) (end 192.363 109.051) (width 0.2) (layer "B.Cu") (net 9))
 (segment (start 199.983 108.40605) (end 199.33805 109.051) (width 0.2) (layer "B.Cu") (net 9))
 (segment (start 198.882 100.33) (end 199.983 101.431) (width 0.2) (layer "B.Cu") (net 9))
 (segment (start 199.983 101.431) (end 199.983 108.40605) (width 0.2) (layer "B.Cu") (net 9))
 (segment (start 193.4972 93.025892) (end 198.882 98.410692) (width 0.2) (layer "B.Cu") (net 9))
 (segment (start 192.363 109.051) (end 191.262 107.95) (width 0.2) (layer "B.Cu") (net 9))
 (segment (start 196.85 124.8156) (end 199.39 124.8156) (width 0.2) (layer "F.Cu") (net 10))
 (segment (start 203.3016 108.6612) (end 203.3016 107.2896) (width 0.2) (layer "F.Cu") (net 10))
 (segment (start 203.3016 107.2896) (end 198.882 102.87) (width 0.2) (layer "F.Cu") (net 10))
 (segment (start 202.3707 109.5921) (end 202.3707 121.8349) (width 0.2) (layer "B.Cu") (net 10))
 (segment (start 202.3707 121.8349) (end 199.39 124.8156) (width 0.2) (layer "B.Cu") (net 10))
 (segment (start 203.3016 108.6612) (end 202.3707 109.5921) (width 0.2) (layer "B.Cu") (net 10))
 (segment (start 200.804 125.9416) (end 195.770735 125.9416) (width 0.2) (layer "F.Cu") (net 11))
 (segment (start 192.8533 112.864165) (end 192.8533 111.4387) (width 0.2) (layer "F.Cu") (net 11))
 (segment (start 195.770735 125.9416) (end 190.3133 120.484165) (width 0.2) (layer "F.Cu") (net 11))
 (segment (start 201.93 124.8156) (end 200.804 125.9416) (width 0.2) (layer "F.Cu") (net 11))
 (segment (start 190.3133 120.484165) (end 190.3133 115.404165) (width 0.2) (layer "F.Cu") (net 11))
 (segment (start 192.8533 111.4387) (end 198.882 105.41) (width 0.2) (layer "F.Cu") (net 11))
 (segment (start 190.3133 115.404165) (end 192.8533 112.864165) (width 0.2) (layer "F.Cu") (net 11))
 (segment (start 191.262 112.4712) (end 190.161 111.3702) (width 0.2) (layer "B.Cu") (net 19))
 (segment (start 190.161 106.511) (end 191.262 105.41) (width 0.2) (layer "B.Cu") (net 19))
 (segment (start 190.161 111.3702) (end 190.161 106.511) (width 0.2) (layer "B.Cu") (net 19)))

